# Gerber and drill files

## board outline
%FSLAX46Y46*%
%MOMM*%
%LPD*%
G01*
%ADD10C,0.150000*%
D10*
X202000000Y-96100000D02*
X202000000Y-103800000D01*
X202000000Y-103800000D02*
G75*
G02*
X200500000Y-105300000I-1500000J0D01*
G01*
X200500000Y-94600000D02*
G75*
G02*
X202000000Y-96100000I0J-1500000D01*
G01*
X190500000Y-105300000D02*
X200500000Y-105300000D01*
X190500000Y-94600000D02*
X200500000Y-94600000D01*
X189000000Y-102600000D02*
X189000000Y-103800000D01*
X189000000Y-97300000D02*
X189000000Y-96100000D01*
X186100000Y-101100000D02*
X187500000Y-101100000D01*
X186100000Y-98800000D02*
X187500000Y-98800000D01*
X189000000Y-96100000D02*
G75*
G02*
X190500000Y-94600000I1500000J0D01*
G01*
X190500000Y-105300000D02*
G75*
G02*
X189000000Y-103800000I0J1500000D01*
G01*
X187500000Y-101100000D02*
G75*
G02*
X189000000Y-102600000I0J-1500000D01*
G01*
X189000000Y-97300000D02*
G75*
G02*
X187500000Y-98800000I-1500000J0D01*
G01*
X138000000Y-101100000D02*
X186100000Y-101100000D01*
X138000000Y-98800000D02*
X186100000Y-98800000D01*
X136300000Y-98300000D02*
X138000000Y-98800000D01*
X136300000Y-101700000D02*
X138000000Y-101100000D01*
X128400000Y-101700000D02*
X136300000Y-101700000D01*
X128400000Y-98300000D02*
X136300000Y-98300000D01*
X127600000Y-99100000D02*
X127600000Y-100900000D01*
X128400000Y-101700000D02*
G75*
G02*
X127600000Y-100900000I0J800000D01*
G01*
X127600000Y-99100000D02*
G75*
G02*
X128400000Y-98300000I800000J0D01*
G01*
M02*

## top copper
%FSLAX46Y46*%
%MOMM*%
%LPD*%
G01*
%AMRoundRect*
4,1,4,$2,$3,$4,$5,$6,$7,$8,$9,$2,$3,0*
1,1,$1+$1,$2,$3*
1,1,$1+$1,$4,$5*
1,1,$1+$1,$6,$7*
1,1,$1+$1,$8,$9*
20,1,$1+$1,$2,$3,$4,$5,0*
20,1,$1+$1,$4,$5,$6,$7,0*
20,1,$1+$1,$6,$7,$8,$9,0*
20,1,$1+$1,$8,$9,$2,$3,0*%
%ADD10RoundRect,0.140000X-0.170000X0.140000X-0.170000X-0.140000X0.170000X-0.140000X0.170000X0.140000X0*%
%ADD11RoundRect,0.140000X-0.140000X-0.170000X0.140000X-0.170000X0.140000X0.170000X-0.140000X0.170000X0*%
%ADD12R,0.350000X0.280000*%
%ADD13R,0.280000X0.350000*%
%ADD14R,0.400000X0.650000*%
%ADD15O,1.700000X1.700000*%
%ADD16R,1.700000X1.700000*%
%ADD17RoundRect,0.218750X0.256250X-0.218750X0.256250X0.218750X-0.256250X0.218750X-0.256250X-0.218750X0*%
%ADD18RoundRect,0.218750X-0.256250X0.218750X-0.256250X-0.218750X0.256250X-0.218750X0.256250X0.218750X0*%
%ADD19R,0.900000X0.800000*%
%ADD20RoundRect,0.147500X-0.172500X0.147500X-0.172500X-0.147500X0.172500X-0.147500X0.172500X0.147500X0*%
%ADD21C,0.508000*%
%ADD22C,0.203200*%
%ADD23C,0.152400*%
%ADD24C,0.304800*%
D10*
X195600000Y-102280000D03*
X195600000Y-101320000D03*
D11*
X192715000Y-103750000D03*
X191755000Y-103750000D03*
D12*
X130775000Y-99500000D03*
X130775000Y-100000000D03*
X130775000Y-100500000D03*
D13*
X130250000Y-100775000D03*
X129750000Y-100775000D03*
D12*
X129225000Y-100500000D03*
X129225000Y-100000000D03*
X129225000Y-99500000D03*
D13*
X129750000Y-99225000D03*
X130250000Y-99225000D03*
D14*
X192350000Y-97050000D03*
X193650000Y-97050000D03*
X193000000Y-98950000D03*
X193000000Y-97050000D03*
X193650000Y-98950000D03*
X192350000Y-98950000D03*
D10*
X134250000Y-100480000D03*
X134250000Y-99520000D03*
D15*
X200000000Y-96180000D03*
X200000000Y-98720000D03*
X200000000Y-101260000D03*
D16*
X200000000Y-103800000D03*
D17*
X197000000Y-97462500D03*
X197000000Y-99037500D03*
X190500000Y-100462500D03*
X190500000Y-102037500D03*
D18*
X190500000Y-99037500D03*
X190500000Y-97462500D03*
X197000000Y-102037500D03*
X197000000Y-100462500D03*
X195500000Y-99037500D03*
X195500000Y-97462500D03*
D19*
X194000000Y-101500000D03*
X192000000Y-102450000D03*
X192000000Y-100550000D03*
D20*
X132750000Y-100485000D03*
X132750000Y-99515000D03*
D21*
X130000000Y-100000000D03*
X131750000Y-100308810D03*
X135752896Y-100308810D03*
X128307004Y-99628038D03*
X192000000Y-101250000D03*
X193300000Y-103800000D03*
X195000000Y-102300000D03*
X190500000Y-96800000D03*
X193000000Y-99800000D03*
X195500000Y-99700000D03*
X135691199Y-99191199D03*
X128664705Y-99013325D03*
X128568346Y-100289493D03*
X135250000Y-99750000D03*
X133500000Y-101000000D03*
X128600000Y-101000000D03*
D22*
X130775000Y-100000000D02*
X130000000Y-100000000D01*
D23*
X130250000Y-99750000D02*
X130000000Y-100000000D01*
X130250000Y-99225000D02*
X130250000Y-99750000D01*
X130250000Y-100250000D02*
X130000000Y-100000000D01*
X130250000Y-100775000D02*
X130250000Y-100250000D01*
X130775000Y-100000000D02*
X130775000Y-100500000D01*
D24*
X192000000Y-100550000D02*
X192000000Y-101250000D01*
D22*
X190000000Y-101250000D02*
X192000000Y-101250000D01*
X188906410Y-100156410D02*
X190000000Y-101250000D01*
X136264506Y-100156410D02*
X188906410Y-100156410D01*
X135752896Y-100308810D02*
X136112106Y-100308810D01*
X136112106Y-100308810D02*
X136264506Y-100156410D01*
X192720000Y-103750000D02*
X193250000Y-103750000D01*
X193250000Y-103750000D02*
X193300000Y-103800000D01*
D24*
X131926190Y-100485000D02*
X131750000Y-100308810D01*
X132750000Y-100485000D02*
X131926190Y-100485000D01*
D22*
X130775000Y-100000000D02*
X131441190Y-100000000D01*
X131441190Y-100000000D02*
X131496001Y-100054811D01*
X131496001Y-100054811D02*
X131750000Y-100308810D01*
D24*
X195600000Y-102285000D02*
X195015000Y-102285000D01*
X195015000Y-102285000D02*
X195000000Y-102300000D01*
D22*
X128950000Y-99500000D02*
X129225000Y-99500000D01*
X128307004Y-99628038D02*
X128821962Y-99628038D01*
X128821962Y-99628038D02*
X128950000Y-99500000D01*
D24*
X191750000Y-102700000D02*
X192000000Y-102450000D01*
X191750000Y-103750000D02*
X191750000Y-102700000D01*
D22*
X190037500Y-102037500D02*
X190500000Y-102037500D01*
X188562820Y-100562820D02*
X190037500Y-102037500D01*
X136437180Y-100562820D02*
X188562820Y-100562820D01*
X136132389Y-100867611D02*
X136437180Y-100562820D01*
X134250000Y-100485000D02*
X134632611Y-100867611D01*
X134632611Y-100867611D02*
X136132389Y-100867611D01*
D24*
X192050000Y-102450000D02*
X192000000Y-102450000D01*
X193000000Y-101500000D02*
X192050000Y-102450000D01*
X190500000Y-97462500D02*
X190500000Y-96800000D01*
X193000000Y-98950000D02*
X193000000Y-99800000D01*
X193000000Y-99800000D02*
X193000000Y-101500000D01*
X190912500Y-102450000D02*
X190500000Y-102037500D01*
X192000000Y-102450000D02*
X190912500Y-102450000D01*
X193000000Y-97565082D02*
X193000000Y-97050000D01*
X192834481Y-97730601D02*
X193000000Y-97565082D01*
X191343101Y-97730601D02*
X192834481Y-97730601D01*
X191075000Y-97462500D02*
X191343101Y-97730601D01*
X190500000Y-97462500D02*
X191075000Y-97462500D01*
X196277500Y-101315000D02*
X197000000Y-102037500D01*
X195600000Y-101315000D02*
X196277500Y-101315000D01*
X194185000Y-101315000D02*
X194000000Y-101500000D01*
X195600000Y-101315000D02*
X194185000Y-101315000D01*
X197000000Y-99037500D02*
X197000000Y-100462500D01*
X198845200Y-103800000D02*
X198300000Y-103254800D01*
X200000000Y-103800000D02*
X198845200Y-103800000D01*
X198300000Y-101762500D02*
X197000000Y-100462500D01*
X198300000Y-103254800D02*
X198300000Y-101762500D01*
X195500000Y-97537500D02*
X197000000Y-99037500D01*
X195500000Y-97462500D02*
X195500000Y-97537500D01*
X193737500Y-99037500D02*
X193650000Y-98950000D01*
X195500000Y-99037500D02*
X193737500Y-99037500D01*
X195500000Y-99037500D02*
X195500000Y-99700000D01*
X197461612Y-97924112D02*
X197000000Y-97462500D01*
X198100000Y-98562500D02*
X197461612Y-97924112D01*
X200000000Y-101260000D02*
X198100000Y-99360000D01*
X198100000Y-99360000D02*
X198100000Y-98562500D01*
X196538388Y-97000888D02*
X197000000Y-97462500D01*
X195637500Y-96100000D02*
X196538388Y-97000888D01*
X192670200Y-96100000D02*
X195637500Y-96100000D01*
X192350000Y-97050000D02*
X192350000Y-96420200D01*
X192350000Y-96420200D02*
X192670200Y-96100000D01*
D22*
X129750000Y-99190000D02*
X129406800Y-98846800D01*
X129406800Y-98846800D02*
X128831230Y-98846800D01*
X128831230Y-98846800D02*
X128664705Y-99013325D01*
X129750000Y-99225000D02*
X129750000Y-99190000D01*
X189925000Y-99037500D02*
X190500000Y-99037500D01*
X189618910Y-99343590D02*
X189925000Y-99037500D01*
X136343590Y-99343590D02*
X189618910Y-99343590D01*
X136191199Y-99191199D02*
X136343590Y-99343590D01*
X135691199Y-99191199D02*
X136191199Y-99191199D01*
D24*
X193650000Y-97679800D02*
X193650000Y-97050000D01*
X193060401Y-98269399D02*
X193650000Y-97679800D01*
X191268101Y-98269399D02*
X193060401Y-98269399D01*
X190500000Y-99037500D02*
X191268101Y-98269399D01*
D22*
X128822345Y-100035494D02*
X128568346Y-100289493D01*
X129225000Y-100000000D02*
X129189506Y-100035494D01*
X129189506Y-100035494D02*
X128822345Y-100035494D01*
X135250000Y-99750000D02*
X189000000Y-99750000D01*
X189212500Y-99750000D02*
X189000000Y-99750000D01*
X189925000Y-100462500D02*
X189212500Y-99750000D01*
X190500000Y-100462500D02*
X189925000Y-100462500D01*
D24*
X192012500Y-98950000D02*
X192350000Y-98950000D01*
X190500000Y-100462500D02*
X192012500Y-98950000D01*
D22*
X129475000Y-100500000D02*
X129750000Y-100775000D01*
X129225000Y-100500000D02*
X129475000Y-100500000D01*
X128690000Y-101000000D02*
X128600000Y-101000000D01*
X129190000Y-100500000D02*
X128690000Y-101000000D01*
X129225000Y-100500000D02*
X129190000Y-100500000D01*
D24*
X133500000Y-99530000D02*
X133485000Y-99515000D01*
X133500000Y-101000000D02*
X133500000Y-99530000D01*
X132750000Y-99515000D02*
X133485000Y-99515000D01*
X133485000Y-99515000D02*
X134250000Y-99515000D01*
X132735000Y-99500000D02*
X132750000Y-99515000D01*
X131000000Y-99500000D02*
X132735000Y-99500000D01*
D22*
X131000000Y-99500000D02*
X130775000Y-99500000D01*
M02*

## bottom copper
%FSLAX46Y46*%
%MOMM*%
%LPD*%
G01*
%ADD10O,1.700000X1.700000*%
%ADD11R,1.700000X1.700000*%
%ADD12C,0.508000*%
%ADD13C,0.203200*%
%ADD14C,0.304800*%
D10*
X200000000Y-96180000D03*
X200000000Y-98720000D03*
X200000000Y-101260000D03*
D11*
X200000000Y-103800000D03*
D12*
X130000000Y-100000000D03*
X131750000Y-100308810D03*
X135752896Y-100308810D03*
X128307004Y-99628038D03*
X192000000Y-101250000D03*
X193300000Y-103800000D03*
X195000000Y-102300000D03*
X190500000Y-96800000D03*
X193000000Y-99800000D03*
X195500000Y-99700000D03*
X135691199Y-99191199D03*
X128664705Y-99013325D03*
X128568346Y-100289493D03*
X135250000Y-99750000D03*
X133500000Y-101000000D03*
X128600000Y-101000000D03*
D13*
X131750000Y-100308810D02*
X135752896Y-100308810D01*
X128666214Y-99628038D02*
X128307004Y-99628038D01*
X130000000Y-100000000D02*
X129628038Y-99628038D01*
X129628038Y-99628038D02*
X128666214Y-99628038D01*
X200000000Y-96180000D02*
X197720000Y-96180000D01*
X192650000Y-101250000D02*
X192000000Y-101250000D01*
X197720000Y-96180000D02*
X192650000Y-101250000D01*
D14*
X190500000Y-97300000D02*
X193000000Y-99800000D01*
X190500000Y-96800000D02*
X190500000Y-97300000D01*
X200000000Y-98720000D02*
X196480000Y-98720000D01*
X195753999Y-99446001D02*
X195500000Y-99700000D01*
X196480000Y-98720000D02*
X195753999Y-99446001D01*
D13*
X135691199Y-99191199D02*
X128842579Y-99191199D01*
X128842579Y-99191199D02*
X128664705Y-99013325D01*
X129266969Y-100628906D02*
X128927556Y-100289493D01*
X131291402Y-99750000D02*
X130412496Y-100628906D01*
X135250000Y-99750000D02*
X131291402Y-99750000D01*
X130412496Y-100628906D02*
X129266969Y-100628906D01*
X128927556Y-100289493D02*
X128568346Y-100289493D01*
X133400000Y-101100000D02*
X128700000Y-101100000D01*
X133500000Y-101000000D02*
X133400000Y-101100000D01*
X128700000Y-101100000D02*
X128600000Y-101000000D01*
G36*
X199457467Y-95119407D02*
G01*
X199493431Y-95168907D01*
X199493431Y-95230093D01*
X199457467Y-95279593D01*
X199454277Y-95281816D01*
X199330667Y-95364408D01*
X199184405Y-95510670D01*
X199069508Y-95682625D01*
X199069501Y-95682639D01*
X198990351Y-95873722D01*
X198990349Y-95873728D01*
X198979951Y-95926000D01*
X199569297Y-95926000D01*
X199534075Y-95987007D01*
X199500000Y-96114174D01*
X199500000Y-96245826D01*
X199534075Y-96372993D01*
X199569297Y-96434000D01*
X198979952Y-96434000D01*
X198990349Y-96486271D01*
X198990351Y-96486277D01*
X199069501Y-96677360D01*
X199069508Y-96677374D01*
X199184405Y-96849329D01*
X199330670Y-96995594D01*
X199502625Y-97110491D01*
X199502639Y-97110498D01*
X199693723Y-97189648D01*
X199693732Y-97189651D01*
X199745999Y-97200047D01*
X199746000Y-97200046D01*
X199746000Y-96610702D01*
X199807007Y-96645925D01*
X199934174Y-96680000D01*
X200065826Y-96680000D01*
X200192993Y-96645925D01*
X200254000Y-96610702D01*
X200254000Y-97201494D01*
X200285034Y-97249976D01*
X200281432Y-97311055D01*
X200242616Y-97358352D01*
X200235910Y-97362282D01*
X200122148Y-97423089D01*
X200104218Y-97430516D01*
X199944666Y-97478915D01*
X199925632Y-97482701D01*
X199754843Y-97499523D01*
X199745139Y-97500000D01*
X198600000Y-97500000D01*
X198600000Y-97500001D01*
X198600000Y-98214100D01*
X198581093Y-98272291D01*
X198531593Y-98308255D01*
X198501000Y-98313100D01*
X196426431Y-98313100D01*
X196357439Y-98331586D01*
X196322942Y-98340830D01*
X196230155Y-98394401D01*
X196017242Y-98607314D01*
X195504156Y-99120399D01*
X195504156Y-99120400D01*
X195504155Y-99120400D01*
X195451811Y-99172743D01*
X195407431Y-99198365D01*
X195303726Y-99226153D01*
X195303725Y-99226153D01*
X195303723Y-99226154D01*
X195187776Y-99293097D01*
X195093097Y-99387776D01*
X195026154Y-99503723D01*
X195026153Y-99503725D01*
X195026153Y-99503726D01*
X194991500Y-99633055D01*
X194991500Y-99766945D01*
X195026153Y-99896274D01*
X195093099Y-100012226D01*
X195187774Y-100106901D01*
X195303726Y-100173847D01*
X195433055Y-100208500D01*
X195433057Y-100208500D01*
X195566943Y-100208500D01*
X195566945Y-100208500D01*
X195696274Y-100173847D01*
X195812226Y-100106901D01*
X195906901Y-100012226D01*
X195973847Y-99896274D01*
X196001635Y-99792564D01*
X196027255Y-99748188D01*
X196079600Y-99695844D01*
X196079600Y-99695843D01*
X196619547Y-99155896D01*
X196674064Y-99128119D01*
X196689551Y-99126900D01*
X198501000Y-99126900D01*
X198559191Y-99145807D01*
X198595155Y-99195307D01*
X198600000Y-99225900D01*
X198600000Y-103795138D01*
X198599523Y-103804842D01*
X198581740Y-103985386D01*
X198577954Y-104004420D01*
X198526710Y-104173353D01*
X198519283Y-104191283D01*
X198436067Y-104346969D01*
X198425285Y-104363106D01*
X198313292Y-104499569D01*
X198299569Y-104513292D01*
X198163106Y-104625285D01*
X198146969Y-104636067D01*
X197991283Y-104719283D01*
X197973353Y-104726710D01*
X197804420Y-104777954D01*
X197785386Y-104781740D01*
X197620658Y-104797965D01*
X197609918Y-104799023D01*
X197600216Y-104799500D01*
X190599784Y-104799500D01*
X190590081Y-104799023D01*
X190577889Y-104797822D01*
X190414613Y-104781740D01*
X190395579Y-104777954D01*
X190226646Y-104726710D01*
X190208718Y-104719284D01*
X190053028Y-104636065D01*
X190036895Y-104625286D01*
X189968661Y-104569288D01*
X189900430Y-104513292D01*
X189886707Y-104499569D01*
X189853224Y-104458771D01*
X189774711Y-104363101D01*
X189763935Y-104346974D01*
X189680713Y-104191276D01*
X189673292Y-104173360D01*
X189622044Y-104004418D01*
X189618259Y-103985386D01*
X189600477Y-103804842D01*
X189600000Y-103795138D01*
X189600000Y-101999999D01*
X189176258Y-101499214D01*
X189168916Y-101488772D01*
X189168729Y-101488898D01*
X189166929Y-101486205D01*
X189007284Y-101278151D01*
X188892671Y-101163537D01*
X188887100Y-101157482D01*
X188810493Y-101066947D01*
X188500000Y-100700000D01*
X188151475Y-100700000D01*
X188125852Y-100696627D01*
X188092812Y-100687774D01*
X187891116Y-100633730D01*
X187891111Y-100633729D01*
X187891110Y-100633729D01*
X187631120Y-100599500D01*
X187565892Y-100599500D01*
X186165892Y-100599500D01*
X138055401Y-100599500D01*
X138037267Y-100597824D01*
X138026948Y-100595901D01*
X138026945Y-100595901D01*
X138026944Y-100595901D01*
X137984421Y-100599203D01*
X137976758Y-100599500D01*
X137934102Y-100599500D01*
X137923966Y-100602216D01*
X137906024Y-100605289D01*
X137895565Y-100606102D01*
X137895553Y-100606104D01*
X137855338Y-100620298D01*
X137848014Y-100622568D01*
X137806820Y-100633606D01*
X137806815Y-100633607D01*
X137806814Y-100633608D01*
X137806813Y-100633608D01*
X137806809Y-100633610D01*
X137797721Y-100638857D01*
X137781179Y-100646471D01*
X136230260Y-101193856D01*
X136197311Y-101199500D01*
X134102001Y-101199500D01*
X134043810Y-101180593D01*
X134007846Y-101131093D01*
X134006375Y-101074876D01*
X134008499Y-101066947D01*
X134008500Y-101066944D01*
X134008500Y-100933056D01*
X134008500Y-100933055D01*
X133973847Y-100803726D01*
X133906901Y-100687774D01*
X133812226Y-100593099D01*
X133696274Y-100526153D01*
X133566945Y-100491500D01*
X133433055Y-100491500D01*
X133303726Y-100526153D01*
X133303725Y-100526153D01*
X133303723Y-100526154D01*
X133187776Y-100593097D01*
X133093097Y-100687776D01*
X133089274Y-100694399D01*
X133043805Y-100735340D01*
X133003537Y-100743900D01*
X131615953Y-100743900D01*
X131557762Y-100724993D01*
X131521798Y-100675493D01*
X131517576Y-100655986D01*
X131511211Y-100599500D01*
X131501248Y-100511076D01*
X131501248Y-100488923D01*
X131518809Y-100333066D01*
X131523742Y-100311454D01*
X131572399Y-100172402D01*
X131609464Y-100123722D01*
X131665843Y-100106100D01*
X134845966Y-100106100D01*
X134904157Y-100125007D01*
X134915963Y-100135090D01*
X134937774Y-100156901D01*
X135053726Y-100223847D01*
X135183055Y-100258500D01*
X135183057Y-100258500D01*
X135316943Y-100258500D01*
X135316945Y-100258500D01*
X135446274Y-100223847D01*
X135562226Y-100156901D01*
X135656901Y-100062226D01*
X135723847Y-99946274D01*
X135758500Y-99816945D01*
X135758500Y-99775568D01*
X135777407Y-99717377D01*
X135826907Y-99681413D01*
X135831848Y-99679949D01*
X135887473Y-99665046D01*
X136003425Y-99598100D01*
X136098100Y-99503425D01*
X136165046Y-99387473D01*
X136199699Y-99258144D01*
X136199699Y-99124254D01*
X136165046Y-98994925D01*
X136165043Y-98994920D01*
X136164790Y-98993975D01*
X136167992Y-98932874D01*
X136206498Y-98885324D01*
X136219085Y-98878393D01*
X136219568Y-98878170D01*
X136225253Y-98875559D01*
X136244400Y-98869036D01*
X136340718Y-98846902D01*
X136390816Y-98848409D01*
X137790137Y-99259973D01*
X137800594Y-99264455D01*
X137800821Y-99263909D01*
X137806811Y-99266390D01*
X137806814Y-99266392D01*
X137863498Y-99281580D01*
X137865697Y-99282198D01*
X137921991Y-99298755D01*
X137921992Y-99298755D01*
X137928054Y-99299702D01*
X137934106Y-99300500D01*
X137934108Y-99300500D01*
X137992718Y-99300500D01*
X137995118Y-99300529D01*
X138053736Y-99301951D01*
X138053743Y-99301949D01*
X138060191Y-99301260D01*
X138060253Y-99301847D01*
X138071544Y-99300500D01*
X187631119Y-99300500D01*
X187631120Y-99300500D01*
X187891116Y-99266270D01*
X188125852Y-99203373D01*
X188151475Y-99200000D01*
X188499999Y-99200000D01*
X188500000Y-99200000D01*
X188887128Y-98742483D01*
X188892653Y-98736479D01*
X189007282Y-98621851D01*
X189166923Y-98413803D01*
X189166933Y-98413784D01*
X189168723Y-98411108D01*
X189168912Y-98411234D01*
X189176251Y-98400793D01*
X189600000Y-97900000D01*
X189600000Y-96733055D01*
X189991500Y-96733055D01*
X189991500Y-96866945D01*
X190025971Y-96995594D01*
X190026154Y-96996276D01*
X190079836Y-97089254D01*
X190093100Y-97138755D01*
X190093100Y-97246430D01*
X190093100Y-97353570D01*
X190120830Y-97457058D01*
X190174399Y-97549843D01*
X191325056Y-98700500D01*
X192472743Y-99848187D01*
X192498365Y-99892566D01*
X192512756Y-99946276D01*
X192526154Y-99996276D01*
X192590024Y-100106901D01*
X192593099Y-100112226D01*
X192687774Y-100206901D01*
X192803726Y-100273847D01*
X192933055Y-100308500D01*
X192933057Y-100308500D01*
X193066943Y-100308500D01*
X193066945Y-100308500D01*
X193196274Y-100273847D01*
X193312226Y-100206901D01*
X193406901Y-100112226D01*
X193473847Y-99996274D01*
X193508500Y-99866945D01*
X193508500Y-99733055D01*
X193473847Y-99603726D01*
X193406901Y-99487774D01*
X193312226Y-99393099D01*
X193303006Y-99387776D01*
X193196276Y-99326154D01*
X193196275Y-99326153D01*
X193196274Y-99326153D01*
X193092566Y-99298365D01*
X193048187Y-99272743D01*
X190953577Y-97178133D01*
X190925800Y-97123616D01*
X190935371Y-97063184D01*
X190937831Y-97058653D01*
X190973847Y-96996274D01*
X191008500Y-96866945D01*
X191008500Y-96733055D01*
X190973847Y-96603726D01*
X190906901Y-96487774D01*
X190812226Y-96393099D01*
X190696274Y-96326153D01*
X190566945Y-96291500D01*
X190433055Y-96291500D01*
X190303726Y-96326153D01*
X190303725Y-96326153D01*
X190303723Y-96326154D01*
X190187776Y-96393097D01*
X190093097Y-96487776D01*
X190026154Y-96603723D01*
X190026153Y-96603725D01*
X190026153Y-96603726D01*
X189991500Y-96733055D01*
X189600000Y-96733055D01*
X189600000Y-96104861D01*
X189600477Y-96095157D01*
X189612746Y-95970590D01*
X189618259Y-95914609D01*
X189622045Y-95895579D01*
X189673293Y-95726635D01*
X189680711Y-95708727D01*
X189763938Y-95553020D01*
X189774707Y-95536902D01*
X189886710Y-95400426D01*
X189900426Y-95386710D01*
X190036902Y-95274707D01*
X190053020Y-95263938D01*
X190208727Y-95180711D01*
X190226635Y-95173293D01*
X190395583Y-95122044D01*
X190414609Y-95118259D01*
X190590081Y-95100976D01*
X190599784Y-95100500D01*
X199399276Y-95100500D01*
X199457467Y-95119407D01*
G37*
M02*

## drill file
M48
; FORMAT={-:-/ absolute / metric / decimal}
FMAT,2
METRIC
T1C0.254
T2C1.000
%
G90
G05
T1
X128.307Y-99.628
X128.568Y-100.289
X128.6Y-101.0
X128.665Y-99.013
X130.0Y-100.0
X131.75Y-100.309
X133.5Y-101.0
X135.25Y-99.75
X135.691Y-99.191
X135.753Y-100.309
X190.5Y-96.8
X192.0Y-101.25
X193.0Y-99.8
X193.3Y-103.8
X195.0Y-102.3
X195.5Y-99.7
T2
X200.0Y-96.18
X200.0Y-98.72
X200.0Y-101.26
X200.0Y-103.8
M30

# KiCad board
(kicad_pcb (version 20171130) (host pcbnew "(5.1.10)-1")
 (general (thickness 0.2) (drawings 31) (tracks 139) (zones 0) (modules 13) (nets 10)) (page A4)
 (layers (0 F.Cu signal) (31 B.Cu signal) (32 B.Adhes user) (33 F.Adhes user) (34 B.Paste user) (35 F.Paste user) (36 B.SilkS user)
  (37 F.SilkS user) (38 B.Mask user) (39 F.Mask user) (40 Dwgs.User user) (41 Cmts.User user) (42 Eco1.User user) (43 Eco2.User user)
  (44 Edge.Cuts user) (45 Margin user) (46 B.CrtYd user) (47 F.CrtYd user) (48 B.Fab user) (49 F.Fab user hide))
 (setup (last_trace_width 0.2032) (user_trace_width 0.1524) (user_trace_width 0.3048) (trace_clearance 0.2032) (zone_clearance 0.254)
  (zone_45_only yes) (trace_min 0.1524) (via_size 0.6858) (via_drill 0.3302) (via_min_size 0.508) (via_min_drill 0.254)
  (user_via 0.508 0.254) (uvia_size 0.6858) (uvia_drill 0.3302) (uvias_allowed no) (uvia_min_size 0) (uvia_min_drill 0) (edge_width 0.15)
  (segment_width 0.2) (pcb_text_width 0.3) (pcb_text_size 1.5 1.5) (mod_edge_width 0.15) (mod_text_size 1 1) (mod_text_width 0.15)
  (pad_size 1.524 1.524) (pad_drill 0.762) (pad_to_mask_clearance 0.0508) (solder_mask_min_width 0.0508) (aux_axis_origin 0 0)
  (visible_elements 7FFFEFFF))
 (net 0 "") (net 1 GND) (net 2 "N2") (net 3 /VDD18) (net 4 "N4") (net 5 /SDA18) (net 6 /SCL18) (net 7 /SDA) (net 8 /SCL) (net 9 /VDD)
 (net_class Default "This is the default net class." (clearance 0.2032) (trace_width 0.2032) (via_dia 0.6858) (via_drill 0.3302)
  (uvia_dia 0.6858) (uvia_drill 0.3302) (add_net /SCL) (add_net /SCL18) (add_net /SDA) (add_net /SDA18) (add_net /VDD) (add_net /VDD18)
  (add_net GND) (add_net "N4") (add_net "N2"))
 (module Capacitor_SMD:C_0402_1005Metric (layer F.Cu) (at 195.6 101.8 270)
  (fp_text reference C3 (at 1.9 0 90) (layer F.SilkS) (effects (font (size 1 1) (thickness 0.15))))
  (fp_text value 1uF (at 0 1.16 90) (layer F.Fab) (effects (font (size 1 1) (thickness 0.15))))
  (pad 2 smd roundrect (at 0.48 0 270) (size 0.56 0.62) (layers F.Cu F.Paste F.Mask) (roundrect_rratio 0.25) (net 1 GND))
  (pad 1 smd roundrect (at -0.48 0 270) (size 0.56 0.62) (layers F.Cu F.Paste F.Mask) (roundrect_rratio 0.25) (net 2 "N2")))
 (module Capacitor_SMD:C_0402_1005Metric (layer F.Cu) (at 192.235 103.75)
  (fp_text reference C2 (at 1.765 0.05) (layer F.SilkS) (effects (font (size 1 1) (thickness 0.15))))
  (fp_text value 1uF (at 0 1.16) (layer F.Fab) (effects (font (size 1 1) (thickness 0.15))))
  (pad 2 smd roundrect (at 0.48 0) (size 0.56 0.62) (layers F.Cu F.Paste F.Mask) (roundrect_rratio 0.25) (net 1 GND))
  (pad 1 smd roundrect (at -0.48 0) (size 0.56 0.62) (layers F.Cu F.Paste F.Mask) (roundrect_rratio 0.25) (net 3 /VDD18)))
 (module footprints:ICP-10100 (layer F.Cu) (at 130 100 270)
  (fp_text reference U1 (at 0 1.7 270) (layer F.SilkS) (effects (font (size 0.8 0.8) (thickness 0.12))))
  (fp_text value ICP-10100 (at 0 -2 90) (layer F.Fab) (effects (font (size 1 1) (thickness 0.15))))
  (pad 10 smd rect (at -0.5 -0.775 270) (size 0.28 0.35) (layers F.Cu F.Paste F.Mask) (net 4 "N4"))
  (pad 9 smd rect (at 0 -0.775 270) (size 0.28 0.35) (layers F.Cu F.Paste F.Mask) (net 1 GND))
  (pad 8 smd rect (at 0.5 -0.775 90) (size 0.28 0.35) (layers F.Cu F.Paste F.Mask) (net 1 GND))
  (pad 7 smd rect (at 0.775 -0.25) (size 0.28 0.35) (layers F.Cu F.Paste F.Mask) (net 1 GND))
  (pad 6 smd rect (at 0.775 0.25) (size 0.28 0.35) (layers F.Cu F.Paste F.Mask) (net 4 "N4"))
  (pad 5 smd rect (at 0.5 0.775 270) (size 0.28 0.35) (layers F.Cu F.Paste F.Mask) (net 4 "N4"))
  (pad 4 smd rect (at 0 0.775 270) (size 0.28 0.35) (layers F.Cu F.Paste F.Mask) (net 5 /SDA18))
  (pad 3 smd rect (at -0.5 0.775 270) (size 0.28 0.35) (layers F.Cu F.Paste F.Mask) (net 1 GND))
  (pad 2 smd rect (at -0.775 0.25) (size 0.28 0.35) (layers F.Cu F.Paste F.Mask) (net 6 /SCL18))
  (pad 1 smd rect (at -0.775 -0.25) (size 0.28 0.35) (layers F.Cu F.Paste F.Mask) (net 1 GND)))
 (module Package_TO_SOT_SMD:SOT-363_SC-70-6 (layer F.Cu) (at 193 98 90)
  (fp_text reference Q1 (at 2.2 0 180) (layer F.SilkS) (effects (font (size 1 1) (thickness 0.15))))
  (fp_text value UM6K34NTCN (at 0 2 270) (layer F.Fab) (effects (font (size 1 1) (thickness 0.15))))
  (pad 6 smd rect (at 0.95 -0.65 90) (size 0.65 0.4) (layers F.Cu F.Paste F.Mask) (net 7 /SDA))
  (pad 4 smd rect (at 0.95 0.65 90) (size 0.65 0.4) (layers F.Cu F.Paste F.Mask) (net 6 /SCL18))
  (pad 2 smd rect (at -0.95 0 90) (size 0.65 0.4) (layers F.Cu F.Paste F.Mask) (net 3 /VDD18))
  (pad 5 smd rect (at 0.95 0 90) (size 0.65 0.4) (layers F.Cu F.Paste F.Mask) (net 3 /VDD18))
  (pad 3 smd rect (at -0.95 0.65 90) (size 0.65 0.4) (layers F.Cu F.Paste F.Mask) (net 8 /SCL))
  (pad 1 smd rect (at -0.95 -0.65 90) (size 0.65 0.4) (layers F.Cu F.Paste F.Mask) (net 5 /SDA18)))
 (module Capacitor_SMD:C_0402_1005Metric (layer F.Cu) (at 134.25 100 270)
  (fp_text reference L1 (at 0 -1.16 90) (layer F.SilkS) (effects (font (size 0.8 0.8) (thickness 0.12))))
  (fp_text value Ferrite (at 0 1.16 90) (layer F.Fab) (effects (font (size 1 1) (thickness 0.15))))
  (pad 2 smd roundrect (at 0.48 0 270) (size 0.56 0.62) (layers F.Cu F.Paste F.Mask) (roundrect_rratio 0.25) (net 3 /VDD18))
  (pad 1 smd roundrect (at -0.48 0 270) (size 0.56 0.62) (layers F.Cu F.Paste F.Mask) (roundrect_rratio 0.25) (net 4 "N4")))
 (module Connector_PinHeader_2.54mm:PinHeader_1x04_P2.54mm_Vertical (layer F.Cu) (at 200 103.8 180)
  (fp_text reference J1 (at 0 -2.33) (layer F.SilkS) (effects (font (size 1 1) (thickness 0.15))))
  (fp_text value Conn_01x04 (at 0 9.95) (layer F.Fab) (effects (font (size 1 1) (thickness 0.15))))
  (pad 4 thru_hole oval (at 0 7.62 180) (size 1.7 1.7) (drill 1) (layers *.Cu *.Mask) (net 1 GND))
  (pad 3 thru_hole oval (at 0 5.08 180) (size 1.7 1.7) (drill 1) (layers *.Cu *.Mask) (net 8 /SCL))
  (pad 2 thru_hole oval (at 0 2.54 180) (size 1.7 1.7) (drill 1) (layers *.Cu *.Mask) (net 7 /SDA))
  (pad 1 thru_hole rect (at 0 0 180) (size 1.7 1.7) (drill 1) (layers *.Cu *.Mask) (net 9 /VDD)))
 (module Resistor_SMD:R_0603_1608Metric (layer F.Cu) (at 197 98.25 90)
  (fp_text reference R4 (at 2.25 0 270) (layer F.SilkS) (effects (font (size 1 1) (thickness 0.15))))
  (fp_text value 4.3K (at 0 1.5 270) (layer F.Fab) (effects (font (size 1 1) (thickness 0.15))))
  (pad 2 smd roundrect (at 0.7875 0 90) (size 0.875 0.95) (layers F.Cu F.Paste F.Mask) (roundrect_rratio 0.25) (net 7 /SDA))
  (pad 1 smd roundrect (at -0.7875 0 90) (size 0.875 0.95) (layers F.Cu F.Paste F.Mask) (roundrect_rratio 0.25) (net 9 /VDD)))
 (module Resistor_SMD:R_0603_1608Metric (layer F.Cu) (at 190.5 101.25 90)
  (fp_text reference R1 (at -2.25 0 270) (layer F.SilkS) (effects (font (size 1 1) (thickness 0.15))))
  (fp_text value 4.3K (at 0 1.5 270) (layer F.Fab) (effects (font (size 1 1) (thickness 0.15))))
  (pad 2 smd roundrect (at 0.7875 0 90) (size 0.875 0.95) (layers F.Cu F.Paste F.Mask) (roundrect_rratio 0.25) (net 5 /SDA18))
  (pad 1 smd roundrect (at -0.7875 0 90) (size 0.875 0.95) (layers F.Cu F.Paste F.Mask) (roundrect_rratio 0.25) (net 3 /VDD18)))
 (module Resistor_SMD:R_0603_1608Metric (layer F.Cu) (at 190.5 98.25 270)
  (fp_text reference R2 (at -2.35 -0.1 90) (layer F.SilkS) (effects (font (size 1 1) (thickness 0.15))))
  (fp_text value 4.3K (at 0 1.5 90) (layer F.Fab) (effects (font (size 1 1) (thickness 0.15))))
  (pad 2 smd roundrect (at 0.7875 0 270) (size 0.875 0.95) (layers F.Cu F.Paste F.Mask) (roundrect_rratio 0.25) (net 6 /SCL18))
  (pad 1 smd roundrect (at -0.7875 0 270) (size 0.875 0.95) (layers F.Cu F.Paste F.Mask) (roundrect_rratio 0.25) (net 3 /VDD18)))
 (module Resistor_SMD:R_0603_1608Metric (layer F.Cu) (at 197 101.25 270)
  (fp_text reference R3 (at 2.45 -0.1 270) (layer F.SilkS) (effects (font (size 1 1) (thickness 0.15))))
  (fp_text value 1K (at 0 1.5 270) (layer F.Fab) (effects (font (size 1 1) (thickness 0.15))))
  (pad 2 smd roundrect (at 0.7875 0 270) (size 0.875 0.95) (layers F.Cu F.Paste F.Mask) (roundrect_rratio 0.25) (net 2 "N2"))
  (pad 1 smd roundrect (at -0.7875 0 270) (size 0.875 0.95) (layers F.Cu F.Paste F.Mask) (roundrect_rratio 0.25) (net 9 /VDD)))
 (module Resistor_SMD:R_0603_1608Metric (layer F.Cu) (at 195.5 98.25 270)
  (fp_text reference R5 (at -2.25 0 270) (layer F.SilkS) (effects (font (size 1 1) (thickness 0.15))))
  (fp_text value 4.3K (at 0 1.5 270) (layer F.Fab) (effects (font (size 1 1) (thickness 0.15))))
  (pad 2 smd roundrect (at 0.7875 0 270) (size 0.875 0.95) (layers F.Cu F.Paste F.Mask) (roundrect_rratio 0.25) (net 8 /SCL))
  (pad 1 smd roundrect (at -0.7875 0 270) (size 0.875 0.95) (layers F.Cu F.Paste F.Mask) (roundrect_rratio 0.25) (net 9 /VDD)))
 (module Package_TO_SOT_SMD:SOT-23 (layer F.Cu) (at 193 101.5)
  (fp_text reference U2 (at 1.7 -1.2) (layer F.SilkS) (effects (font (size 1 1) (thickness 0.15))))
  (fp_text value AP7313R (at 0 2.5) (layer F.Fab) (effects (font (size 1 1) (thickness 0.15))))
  (pad 3 smd rect (at 1 0) (size 0.9 0.8) (layers F.Cu F.Paste F.Mask) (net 2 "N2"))
  (pad 2 smd rect (at -1 0.95) (size 0.9 0.8) (layers F.Cu F.Paste F.Mask) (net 3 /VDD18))
  (pad 1 smd rect (at -1 -0.95) (size 0.9 0.8) (layers F.Cu F.Paste F.Mask) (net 1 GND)))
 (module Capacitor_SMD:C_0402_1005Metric (layer F.Cu) (at 132.75 100 270)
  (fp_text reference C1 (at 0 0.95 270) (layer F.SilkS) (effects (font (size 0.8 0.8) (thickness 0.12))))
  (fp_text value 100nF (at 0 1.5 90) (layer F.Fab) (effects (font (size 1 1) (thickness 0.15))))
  (pad 2 smd roundrect (at 0.485 0 270) (size 0.59 0.64) (layers F.Cu F.Paste F.Mask) (roundrect_rratio 0.25) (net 1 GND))
  (pad 1 smd roundrect (at -0.485 0 270) (size 0.59 0.64) (layers F.Cu F.Paste F.Mask) (roundrect_rratio 0.25) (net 4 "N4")))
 (gr_line (start 202 96.1) (end 202 103.8) (layer Edge.Cuts) (width 0.15))
 (gr_arc (start 200.5 103.8) (end 200.5 105.3) (angle -90) (layer Edge.Cuts) (width 0.15))
 (gr_arc (start 200.5 96.1) (end 202 96.1) (angle -90) (layer Edge.Cuts) (width 0.15))
 (gr_line (start 190.5 105.3) (end 200.5 105.3) (layer Edge.Cuts) (width 0.15))
 (gr_line (start 190.5 94.6) (end 200.5 94.6) (layer Edge.Cuts) (width 0.15))
 (gr_line (start 189 102.6) (end 189 103.8) (layer Edge.Cuts) (width 0.15))
 (gr_line (start 189 97.3) (end 189 96.1) (layer Edge.Cuts) (width 0.15))
 (gr_line (start 186.1 101.1) (end 187.5 101.1) (layer Edge.Cuts) (width 0.15))
 (gr_line (start 186.1 98.8) (end 187.5 98.8) (layer Edge.Cuts) (width 0.15))
 (gr_arc (start 190.5 96.1) (end 190.5 94.6) (angle -90) (layer Edge.Cuts) (width 0.15))
 (gr_arc (start 190.5 103.8) (end 189 103.8) (angle -90) (layer Edge.Cuts) (width 0.15))
 (gr_arc (start 187.5 102.6) (end 189 102.6) (angle -90) (layer Edge.Cuts) (width 0.15))
 (gr_arc (start 187.5 97.3) (end 187.5 98.8) (angle -90) (layer Edge.Cuts) (width 0.15))
 (gr_line (start 138 101.1) (end 186.1 101.1) (layer Edge.Cuts) (width 0.15))
 (gr_line (start 138 98.8) (end 186.1 98.8) (layer Edge.Cuts) (width 0.15))
 (gr_line (start 136.3 98.3) (end 138 98.8) (layer Edge.Cuts) (width 0.15))
 (gr_line (start 136.3 101.7) (end 138 101.1) (layer Edge.Cuts) (width 0.15))
 (gr_line (start 128.4 101.7) (end 136.3 101.7) (layer Edge.Cuts) (width 0.15))
 (gr_line (start 128.4 98.3) (end 136.3 98.3) (layer Edge.Cuts) (width 0.15))
 (gr_line (start 127.6 99.1) (end 127.6 100.9) (layer Edge.Cuts) (width 0.15))
 (gr_arc (start 128.4 100.9) (end 127.6 100.9) (angle -90) (layer Edge.Cuts) (width 0.15))
 (gr_arc (start 128.4 99.1) (end 128.4 98.3) (angle -90) (layer Edge.Cuts) (width 0.15))
 (segment (start 130.775 100) (end 130 100) (width 0.2032) (layer F.Cu) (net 1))
 (segment (start 130.25 99.75) (end 130 100) (width 0.1524) (layer F.Cu) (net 1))
 (segment (start 130.25 99.225) (end 130.25 99.75) (width 0.1524) (layer F.Cu) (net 1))
 (segment (start 130.25 100.25) (end 130 100) (width 0.1524) (layer F.Cu) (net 1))
 (segment (start 130.25 100.775) (end 130.25 100.25) (width 0.1524) (layer F.Cu) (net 1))
 (segment (start 130.775 100) (end 130.775 100.5) (width 0.1524) (layer F.Cu) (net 1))
 (via (at 130 100) (size 0.508) (drill 0.254) (layers F.Cu B.Cu) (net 1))
 (via (at 131.75 100.30881) (size 0.508) (drill 0.254) (layers F.Cu B.Cu) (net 1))
 (segment (start 131.75 100.30881) (end 135.752896 100.30881) (width 0.2032) (layer B.Cu) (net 1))
 (via (at 135.752896 100.30881) (size 0.508) (drill 0.254) (layers F.Cu B.Cu) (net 1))
 (via (at 128.307004 99.628038) (size 0.508) (drill 0.254) (layers F.Cu B.Cu) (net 1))
 (segment (start 128.666214 99.628038) (end 128.307004 99.628038) (width 0.2032) (layer B.Cu) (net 1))
 (segment (start 130 100) (end 129.628038 99.628038) (width 0.2032) (layer B.Cu) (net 1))
 (segment (start 129.628038 99.628038) (end 128.666214 99.628038) (width 0.2032) (layer B.Cu) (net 1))
 (via (at 192 101.25) (size 0.508) (drill 0.254) (layers F.Cu B.Cu) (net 1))
 (segment (start 192 100.55) (end 192 101.25) (width 0.3048) (layer F.Cu) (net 1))
 (segment (start 190 101.25) (end 192 101.25) (width 0.2032) (layer F.Cu) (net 1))
 (segment (start 188.90641 100.15641) (end 190 101.25) (width 0.2032) (layer F.Cu) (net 1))
 (segment (start 136.264506 100.15641) (end 188.90641 100.15641) (width 0.2032) (layer F.Cu) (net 1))
 (segment (start 135.752896 100.30881) (end 136.112106 100.30881) (width 0.2032) (layer F.Cu) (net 1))
 (segment (start 136.112106 100.30881) (end 136.264506 100.15641) (width 0.2032) (layer F.Cu) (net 1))
 (segment (start 200 96.18) (end 197.72 96.18) (width 0.2032) (layer B.Cu) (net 1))
 (segment (start 192.65 101.25) (end 192 101.25) (width 0.2032) (layer B.Cu) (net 1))
 (segment (start 197.72 96.18) (end 192.65 101.25) (width 0.2032) (layer B.Cu) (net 1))
 (via (at 193.3 103.8) (size 0.508) (drill 0.254) (layers F.Cu B.Cu) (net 1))
 (segment (start 192.72 103.75) (end 193.25 103.75) (width 0.2032) (layer F.Cu) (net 1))
 (segment (start 193.25 103.75) (end 193.3 103.8) (width 0.2032) (layer F.Cu) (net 1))
 (segment (start 131.92619 100.485) (end 131.75 100.30881) (width 0.3048) (layer F.Cu) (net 1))
 (segment (start 132.75 100.485) (end 131.92619 100.485) (width 0.3048) (layer F.Cu) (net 1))
 (segment (start 130.775 100) (end 131.44119 100) (width 0.2032) (layer F.Cu) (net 1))
 (segment (start 131.44119 100) (end 131.496001 100.054811) (width 0.2032) (layer F.Cu) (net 1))
 (segment (start 131.496001 100.054811) (end 131.75 100.30881) (width 0.2032) (layer F.Cu) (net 1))
 (via (at 195 102.3) (size 0.508) (drill 0.254) (layers F.Cu B.Cu) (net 1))
 (segment (start 195.6 102.285) (end 195.015 102.285) (width 0.3048) (layer F.Cu) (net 1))
 (segment (start 195.015 102.285) (end 195 102.3) (width 0.3048) (layer F.Cu) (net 1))
 (segment (start 128.95 99.5) (end 129.225 99.5) (width 0.2032) (layer F.Cu) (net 1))
 (segment (start 128.307004 99.628038) (end 128.821962 99.628038) (width 0.2032) (layer F.Cu) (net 1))
 (segment (start 128.821962 99.628038) (end 128.95 99.5) (width 0.2032) (layer F.Cu) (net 1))
 (segment (start 191.75 102.7) (end 192 102.45) (width 0.3048) (layer F.Cu) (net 3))
 (segment (start 191.75 103.75) (end 191.75 102.7) (width 0.3048) (layer F.Cu) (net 3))
 (segment (start 190.0375 102.0375) (end 190.5 102.0375) (width 0.2032) (layer F.Cu) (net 3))
 (segment (start 188.56282 100.56282) (end 190.0375 102.0375) (width 0.2032) (layer F.Cu) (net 3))
 (segment (start 136.43718 100.56282) (end 188.56282 100.56282) (width 0.2032) (layer F.Cu) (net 3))
 (segment (start 136.132389 100.867611) (end 136.43718 100.56282) (width 0.2032) (layer F.Cu) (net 3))
 (segment (start 134.25 100.485) (end 134.632611 100.867611) (width 0.2032) (layer F.Cu) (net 3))
 (segment (start 134.632611 100.867611) (end 136.132389 100.867611) (width 0.2032) (layer F.Cu) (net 3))
 (segment (start 192.05 102.45) (end 192 102.45) (width 0.3048) (layer F.Cu) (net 3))
 (segment (start 193 101.5) (end 192.05 102.45) (width 0.3048) (layer F.Cu) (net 3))
 (via (at 190.5 96.8) (size 0.508) (drill 0.254) (layers F.Cu B.Cu) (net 3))
 (segment (start 190.5 97.4625) (end 190.5 96.8) (width 0.3048) (layer F.Cu) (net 3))
 (via (at 193 99.8) (size 0.508) (drill 0.254) (layers F.Cu B.Cu) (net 3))
 (segment (start 190.5 97.3) (end 193 99.8) (width 0.3048) (layer B.Cu) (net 3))
 (segment (start 190.5 96.8) (end 190.5 97.3) (width 0.3048) (layer B.Cu) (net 3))
 (segment (start 193 98.95) (end 193 99.8) (width 0.3048) (layer F.Cu) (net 3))
 (segment (start 193 99.8) (end 193 101.5) (width 0.3048) (layer F.Cu) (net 3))
 (segment (start 190.9125 102.45) (end 190.5 102.0375) (width 0.3048) (layer F.Cu) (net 3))
 (segment (start 192 102.45) (end 190.9125 102.45) (width 0.3048) (layer F.Cu) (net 3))
 (segment (start 193 97.565082) (end 193 97.05) (width 0.3048) (layer F.Cu) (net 3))
 (segment (start 192.834481 97.730601) (end 193 97.565082) (width 0.3048) (layer F.Cu) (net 3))
 (segment (start 191.343101 97.730601) (end 192.834481 97.730601) (width 0.3048) (layer F.Cu) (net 3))
 (segment (start 191.075 97.4625) (end 191.343101 97.730601) (width 0.3048) (layer F.Cu) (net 3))
 (segment (start 190.5 97.4625) (end 191.075 97.4625) (width 0.3048) (layer F.Cu) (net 3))
 (segment (start 196.2775 101.315) (end 197 102.0375) (width 0.3048) (layer F.Cu) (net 2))
 (segment (start 195.6 101.315) (end 196.2775 101.315) (width 0.3048) (layer F.Cu) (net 2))
 (segment (start 194.185 101.315) (end 194 101.5) (width 0.3048) (layer F.Cu) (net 2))
 (segment (start 195.6 101.315) (end 194.185 101.315) (width 0.3048) (layer F.Cu) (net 2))
 (segment (start 197 99.0375) (end 197 100.4625) (width 0.3048) (layer F.Cu) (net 9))
 (segment (start 198.8452 103.8) (end 198.3 103.2548) (width 0.3048) (layer F.Cu) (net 9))
 (segment (start 200 103.8) (end 198.8452 103.8) (width 0.3048) (layer F.Cu) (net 9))
 (segment (start 198.3 101.7625) (end 197 100.4625) (width 0.3048) (layer F.Cu) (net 9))
 (segment (start 198.3 103.2548) (end 198.3 101.7625) (width 0.3048) (layer F.Cu) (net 9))
 (segment (start 195.5 97.5375) (end 197 99.0375) (width 0.3048) (layer F.Cu) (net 9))
 (segment (start 195.5 97.4625) (end 195.5 97.5375) (width 0.3048) (layer F.Cu) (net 9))
 (segment (start 193.7375 99.0375) (end 193.65 98.95) (width 0.3048) (layer F.Cu) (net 8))
 (segment (start 195.5 99.0375) (end 193.7375 99.0375) (width 0.3048) (layer F.Cu) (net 8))
 (via (at 195.5 99.7) (size 0.508) (drill 0.254) (layers F.Cu B.Cu) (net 8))
 (segment (start 195.5 99.0375) (end 195.5 99.7) (width 0.3048) (layer F.Cu) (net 8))
 (segment (start 200 98.72) (end 196.48 98.72) (width 0.3048) (layer B.Cu) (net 8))
 (segment (start 195.753999 99.446001) (end 195.5 99.7) (width 0.3048) (layer B.Cu) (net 8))
 (segment (start 196.48 98.72) (end 195.753999 99.446001) (width 0.3048) (layer B.Cu) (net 8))
 (segment (start 197.461612 97.924112) (end 197 97.4625) (width 0.3048) (layer F.Cu) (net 7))
 (segment (start 198.1 98.5625) (end 197.461612 97.924112) (width 0.3048) (layer F.Cu) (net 7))
 (segment (start 200 101.26) (end 198.1 99.36) (width 0.3048) (layer F.Cu) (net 7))
 (segment (start 198.1 99.36) (end 198.1 98.5625) (width 0.3048) (layer F.Cu) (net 7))
 (segment (start 196.538388 97.000888) (end 197 97.4625) (width 0.3048) (layer F.Cu) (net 7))
 (segment (start 195.6375 96.1) (end 196.538388 97.000888) (width 0.3048) (layer F.Cu) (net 7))
 (segment (start 192.6702 96.1) (end 195.6375 96.1) (width 0.3048) (layer F.Cu) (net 7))
 (segment (start 192.35 97.05) (end 192.35 96.4202) (width 0.3048) (layer F.Cu) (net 7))
 (segment (start 192.35 96.4202) (end 192.6702 96.1) (width 0.3048) (layer F.Cu) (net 7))
 (via (at 135.691199 99.191199) (size 0.508) (drill 0.254) (layers F.Cu B.Cu) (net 6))
 (segment (start 129.75 99.19) (end 129.4068 98.8468) (width 0.2032) (layer F.Cu) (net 6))
 (via (at 128.664705 99.013325) (size 0.508) (drill 0.254) (layers F.Cu B.Cu) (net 6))
 (segment (start 129.4068 98.8468) (end 128.83123 98.8468) (width 0.2032) (layer F.Cu) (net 6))
 (segment (start 135.691199 99.191199) (end 128.842579 99.191199) (width 0.2032) (layer B.Cu) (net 6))
 (segment (start 128.83123 98.8468) (end 128.664705 99.013325) (width 0.2032) (layer F.Cu) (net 6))
 (segment (start 128.842579 99.191199) (end 128.664705 99.013325) (width 0.2032) (layer B.Cu) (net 6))
 (segment (start 129.75 99.225) (end 129.75 99.19) (width 0.2032) (layer F.Cu) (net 6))
 (segment (start 189.925 99.0375) (end 190.5 99.0375) (width 0.2032) (layer F.Cu) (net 6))
 (segment (start 189.61891 99.34359) (end 189.925 99.0375) (width 0.2032) (layer F.Cu) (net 6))
 (segment (start 136.34359 99.34359) (end 189.61891 99.34359) (width 0.2032) (layer F.Cu) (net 6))
 (segment (start 136.191199 99.191199) (end 136.34359 99.34359) (width 0.2032) (layer F.Cu) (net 6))
 (segment (start 135.691199 99.191199) (end 136.191199 99.191199) (width 0.2032) (layer F.Cu) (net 6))
 (segment (start 193.65 97.6798) (end 193.65 97.05) (width 0.3048) (layer F.Cu) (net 6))
 (segment (start 193.060401 98.269399) (end 193.65 97.6798) (width 0.3048) (layer F.Cu) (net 6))
 (segment (start 191.268101 98.269399) (end 193.060401 98.269399) (width 0.3048) (layer F.Cu) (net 6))
 (segment (start 190.5 99.0375) (end 191.268101 98.269399) (width 0.3048) (layer F.Cu) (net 6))
 (via (at 128.568346 100.289493) (size 0.508) (drill 0.254) (layers F.Cu B.Cu) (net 5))
 (via (at 135.25 99.75) (size 0.508) (drill 0.254) (layers F.Cu B.Cu) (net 5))
 (segment (start 129.266969 100.628906) (end 128.927556 100.289493) (width 0.2032) (layer B.Cu) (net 5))
 (segment (start 128.822345 100.035494) (end 128.568346 100.289493) (width 0.2032) (layer F.Cu) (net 5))
 (segment (start 129.225 100) (end 129.189506 100.035494) (width 0.2032) (layer F.Cu) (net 5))
 (segment (start 129.189506 100.035494) (end 128.822345 100.035494) (width 0.2032) (layer F.Cu) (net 5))
 (segment (start 131.291402 99.75) (end 130.412496 100.628906) (width 0.2032) (layer B.Cu) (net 5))
 (segment (start 135.25 99.75) (end 131.291402 99.75) (width 0.2032) (layer B.Cu) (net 5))
 (segment (start 130.412496 100.628906) (end 129.266969 100.628906) (width 0.2032) (layer B.Cu) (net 5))
 (segment (start 128.927556 100.289493) (end 128.568346 100.289493) (width 0.2032) (layer B.Cu) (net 5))
 (segment (start 135.25 99.75) (end 189 99.75) (width 0.2032) (layer F.Cu) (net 5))
 (segment (start 189.2125 99.75) (end 189 99.75) (width 0.2032) (layer F.Cu) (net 5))
 (segment (start 189.925 100.4625) (end 189.2125 99.75) (width 0.2032) (layer F.Cu) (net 5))
 (segment (start 190.5 100.4625) (end 189.925 100.4625) (width 0.2032) (layer F.Cu) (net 5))
 (segment (start 192.0125 98.95) (end 192.35 98.95) (width 0.3048) (layer F.Cu) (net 5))
 (segment (start 190.5 100.4625) (end 192.0125 98.95) (width 0.3048) (layer F.Cu) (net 5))
 (segment (start 129.475 100.5) (end 129.75 100.775) (width 0.2032) (layer F.Cu) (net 4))
 (segment (start 129.225 100.5) (end 129.475 100.5) (width 0.2032) (layer F.Cu) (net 4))
 (via (at 133.5 101) (size 0.508) (drill 0.254) (layers F.Cu B.Cu) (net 4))
 (via (at 128.6 101) (size 0.508) (drill 0.254) (layers F.Cu B.Cu) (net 4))
 (segment (start 133.4 101.1) (end 128.7 101.1) (width 0.2032) (layer B.Cu) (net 4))
 (segment (start 133.5 101) (end 133.4 101.1) (width 0.2032) (layer B.Cu) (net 4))
 (segment (start 128.69 101) (end 128.6 101) (width 0.2032) (layer F.Cu) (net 4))
 (segment (start 129.19 100.5) (end 128.69 101) (width 0.2032) (layer F.Cu) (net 4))
 (segment (start 128.7 101.1) (end 128.6 101) (width 0.2032) (layer B.Cu) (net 4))
 (segment (start 129.225 100.5) (end 129.19 100.5) (width 0.2032) (layer F.Cu) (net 4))
 (segment (start 133.5 99.53) (end 133.485 99.515) (width 0.3048) (layer F.Cu) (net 4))
 (segment (start 133.5 101) (end 133.5 99.53) (width 0.3048) (layer F.Cu) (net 4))
 (segment (start 132.75 99.515) (end 133.485 99.515) (width 0.3048) (layer F.Cu) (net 4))
 (segment (start 133.485 99.515) (end 134.25 99.515) (width 0.3048) (layer F.Cu) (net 4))
 (segment (start 132.735 99.5) (end 132.75 99.515) (width 0.3048) (layer F.Cu) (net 4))
 (segment (start 131 99.5) (end 132.735 99.5) (width 0.3048) (layer F.Cu) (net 4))
 (segment (start 131 99.5) (end 130.775 99.5) (width 0.2032) (layer F.Cu) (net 4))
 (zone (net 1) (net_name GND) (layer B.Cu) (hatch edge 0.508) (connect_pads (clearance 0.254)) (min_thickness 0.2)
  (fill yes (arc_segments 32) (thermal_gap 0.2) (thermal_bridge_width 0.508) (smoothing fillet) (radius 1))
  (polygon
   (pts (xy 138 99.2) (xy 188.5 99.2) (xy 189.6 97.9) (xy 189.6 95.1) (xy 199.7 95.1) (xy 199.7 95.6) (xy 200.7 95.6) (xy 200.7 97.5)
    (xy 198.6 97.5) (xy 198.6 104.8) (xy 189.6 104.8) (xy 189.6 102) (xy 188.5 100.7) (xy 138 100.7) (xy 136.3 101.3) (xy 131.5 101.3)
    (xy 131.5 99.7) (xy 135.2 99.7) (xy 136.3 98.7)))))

